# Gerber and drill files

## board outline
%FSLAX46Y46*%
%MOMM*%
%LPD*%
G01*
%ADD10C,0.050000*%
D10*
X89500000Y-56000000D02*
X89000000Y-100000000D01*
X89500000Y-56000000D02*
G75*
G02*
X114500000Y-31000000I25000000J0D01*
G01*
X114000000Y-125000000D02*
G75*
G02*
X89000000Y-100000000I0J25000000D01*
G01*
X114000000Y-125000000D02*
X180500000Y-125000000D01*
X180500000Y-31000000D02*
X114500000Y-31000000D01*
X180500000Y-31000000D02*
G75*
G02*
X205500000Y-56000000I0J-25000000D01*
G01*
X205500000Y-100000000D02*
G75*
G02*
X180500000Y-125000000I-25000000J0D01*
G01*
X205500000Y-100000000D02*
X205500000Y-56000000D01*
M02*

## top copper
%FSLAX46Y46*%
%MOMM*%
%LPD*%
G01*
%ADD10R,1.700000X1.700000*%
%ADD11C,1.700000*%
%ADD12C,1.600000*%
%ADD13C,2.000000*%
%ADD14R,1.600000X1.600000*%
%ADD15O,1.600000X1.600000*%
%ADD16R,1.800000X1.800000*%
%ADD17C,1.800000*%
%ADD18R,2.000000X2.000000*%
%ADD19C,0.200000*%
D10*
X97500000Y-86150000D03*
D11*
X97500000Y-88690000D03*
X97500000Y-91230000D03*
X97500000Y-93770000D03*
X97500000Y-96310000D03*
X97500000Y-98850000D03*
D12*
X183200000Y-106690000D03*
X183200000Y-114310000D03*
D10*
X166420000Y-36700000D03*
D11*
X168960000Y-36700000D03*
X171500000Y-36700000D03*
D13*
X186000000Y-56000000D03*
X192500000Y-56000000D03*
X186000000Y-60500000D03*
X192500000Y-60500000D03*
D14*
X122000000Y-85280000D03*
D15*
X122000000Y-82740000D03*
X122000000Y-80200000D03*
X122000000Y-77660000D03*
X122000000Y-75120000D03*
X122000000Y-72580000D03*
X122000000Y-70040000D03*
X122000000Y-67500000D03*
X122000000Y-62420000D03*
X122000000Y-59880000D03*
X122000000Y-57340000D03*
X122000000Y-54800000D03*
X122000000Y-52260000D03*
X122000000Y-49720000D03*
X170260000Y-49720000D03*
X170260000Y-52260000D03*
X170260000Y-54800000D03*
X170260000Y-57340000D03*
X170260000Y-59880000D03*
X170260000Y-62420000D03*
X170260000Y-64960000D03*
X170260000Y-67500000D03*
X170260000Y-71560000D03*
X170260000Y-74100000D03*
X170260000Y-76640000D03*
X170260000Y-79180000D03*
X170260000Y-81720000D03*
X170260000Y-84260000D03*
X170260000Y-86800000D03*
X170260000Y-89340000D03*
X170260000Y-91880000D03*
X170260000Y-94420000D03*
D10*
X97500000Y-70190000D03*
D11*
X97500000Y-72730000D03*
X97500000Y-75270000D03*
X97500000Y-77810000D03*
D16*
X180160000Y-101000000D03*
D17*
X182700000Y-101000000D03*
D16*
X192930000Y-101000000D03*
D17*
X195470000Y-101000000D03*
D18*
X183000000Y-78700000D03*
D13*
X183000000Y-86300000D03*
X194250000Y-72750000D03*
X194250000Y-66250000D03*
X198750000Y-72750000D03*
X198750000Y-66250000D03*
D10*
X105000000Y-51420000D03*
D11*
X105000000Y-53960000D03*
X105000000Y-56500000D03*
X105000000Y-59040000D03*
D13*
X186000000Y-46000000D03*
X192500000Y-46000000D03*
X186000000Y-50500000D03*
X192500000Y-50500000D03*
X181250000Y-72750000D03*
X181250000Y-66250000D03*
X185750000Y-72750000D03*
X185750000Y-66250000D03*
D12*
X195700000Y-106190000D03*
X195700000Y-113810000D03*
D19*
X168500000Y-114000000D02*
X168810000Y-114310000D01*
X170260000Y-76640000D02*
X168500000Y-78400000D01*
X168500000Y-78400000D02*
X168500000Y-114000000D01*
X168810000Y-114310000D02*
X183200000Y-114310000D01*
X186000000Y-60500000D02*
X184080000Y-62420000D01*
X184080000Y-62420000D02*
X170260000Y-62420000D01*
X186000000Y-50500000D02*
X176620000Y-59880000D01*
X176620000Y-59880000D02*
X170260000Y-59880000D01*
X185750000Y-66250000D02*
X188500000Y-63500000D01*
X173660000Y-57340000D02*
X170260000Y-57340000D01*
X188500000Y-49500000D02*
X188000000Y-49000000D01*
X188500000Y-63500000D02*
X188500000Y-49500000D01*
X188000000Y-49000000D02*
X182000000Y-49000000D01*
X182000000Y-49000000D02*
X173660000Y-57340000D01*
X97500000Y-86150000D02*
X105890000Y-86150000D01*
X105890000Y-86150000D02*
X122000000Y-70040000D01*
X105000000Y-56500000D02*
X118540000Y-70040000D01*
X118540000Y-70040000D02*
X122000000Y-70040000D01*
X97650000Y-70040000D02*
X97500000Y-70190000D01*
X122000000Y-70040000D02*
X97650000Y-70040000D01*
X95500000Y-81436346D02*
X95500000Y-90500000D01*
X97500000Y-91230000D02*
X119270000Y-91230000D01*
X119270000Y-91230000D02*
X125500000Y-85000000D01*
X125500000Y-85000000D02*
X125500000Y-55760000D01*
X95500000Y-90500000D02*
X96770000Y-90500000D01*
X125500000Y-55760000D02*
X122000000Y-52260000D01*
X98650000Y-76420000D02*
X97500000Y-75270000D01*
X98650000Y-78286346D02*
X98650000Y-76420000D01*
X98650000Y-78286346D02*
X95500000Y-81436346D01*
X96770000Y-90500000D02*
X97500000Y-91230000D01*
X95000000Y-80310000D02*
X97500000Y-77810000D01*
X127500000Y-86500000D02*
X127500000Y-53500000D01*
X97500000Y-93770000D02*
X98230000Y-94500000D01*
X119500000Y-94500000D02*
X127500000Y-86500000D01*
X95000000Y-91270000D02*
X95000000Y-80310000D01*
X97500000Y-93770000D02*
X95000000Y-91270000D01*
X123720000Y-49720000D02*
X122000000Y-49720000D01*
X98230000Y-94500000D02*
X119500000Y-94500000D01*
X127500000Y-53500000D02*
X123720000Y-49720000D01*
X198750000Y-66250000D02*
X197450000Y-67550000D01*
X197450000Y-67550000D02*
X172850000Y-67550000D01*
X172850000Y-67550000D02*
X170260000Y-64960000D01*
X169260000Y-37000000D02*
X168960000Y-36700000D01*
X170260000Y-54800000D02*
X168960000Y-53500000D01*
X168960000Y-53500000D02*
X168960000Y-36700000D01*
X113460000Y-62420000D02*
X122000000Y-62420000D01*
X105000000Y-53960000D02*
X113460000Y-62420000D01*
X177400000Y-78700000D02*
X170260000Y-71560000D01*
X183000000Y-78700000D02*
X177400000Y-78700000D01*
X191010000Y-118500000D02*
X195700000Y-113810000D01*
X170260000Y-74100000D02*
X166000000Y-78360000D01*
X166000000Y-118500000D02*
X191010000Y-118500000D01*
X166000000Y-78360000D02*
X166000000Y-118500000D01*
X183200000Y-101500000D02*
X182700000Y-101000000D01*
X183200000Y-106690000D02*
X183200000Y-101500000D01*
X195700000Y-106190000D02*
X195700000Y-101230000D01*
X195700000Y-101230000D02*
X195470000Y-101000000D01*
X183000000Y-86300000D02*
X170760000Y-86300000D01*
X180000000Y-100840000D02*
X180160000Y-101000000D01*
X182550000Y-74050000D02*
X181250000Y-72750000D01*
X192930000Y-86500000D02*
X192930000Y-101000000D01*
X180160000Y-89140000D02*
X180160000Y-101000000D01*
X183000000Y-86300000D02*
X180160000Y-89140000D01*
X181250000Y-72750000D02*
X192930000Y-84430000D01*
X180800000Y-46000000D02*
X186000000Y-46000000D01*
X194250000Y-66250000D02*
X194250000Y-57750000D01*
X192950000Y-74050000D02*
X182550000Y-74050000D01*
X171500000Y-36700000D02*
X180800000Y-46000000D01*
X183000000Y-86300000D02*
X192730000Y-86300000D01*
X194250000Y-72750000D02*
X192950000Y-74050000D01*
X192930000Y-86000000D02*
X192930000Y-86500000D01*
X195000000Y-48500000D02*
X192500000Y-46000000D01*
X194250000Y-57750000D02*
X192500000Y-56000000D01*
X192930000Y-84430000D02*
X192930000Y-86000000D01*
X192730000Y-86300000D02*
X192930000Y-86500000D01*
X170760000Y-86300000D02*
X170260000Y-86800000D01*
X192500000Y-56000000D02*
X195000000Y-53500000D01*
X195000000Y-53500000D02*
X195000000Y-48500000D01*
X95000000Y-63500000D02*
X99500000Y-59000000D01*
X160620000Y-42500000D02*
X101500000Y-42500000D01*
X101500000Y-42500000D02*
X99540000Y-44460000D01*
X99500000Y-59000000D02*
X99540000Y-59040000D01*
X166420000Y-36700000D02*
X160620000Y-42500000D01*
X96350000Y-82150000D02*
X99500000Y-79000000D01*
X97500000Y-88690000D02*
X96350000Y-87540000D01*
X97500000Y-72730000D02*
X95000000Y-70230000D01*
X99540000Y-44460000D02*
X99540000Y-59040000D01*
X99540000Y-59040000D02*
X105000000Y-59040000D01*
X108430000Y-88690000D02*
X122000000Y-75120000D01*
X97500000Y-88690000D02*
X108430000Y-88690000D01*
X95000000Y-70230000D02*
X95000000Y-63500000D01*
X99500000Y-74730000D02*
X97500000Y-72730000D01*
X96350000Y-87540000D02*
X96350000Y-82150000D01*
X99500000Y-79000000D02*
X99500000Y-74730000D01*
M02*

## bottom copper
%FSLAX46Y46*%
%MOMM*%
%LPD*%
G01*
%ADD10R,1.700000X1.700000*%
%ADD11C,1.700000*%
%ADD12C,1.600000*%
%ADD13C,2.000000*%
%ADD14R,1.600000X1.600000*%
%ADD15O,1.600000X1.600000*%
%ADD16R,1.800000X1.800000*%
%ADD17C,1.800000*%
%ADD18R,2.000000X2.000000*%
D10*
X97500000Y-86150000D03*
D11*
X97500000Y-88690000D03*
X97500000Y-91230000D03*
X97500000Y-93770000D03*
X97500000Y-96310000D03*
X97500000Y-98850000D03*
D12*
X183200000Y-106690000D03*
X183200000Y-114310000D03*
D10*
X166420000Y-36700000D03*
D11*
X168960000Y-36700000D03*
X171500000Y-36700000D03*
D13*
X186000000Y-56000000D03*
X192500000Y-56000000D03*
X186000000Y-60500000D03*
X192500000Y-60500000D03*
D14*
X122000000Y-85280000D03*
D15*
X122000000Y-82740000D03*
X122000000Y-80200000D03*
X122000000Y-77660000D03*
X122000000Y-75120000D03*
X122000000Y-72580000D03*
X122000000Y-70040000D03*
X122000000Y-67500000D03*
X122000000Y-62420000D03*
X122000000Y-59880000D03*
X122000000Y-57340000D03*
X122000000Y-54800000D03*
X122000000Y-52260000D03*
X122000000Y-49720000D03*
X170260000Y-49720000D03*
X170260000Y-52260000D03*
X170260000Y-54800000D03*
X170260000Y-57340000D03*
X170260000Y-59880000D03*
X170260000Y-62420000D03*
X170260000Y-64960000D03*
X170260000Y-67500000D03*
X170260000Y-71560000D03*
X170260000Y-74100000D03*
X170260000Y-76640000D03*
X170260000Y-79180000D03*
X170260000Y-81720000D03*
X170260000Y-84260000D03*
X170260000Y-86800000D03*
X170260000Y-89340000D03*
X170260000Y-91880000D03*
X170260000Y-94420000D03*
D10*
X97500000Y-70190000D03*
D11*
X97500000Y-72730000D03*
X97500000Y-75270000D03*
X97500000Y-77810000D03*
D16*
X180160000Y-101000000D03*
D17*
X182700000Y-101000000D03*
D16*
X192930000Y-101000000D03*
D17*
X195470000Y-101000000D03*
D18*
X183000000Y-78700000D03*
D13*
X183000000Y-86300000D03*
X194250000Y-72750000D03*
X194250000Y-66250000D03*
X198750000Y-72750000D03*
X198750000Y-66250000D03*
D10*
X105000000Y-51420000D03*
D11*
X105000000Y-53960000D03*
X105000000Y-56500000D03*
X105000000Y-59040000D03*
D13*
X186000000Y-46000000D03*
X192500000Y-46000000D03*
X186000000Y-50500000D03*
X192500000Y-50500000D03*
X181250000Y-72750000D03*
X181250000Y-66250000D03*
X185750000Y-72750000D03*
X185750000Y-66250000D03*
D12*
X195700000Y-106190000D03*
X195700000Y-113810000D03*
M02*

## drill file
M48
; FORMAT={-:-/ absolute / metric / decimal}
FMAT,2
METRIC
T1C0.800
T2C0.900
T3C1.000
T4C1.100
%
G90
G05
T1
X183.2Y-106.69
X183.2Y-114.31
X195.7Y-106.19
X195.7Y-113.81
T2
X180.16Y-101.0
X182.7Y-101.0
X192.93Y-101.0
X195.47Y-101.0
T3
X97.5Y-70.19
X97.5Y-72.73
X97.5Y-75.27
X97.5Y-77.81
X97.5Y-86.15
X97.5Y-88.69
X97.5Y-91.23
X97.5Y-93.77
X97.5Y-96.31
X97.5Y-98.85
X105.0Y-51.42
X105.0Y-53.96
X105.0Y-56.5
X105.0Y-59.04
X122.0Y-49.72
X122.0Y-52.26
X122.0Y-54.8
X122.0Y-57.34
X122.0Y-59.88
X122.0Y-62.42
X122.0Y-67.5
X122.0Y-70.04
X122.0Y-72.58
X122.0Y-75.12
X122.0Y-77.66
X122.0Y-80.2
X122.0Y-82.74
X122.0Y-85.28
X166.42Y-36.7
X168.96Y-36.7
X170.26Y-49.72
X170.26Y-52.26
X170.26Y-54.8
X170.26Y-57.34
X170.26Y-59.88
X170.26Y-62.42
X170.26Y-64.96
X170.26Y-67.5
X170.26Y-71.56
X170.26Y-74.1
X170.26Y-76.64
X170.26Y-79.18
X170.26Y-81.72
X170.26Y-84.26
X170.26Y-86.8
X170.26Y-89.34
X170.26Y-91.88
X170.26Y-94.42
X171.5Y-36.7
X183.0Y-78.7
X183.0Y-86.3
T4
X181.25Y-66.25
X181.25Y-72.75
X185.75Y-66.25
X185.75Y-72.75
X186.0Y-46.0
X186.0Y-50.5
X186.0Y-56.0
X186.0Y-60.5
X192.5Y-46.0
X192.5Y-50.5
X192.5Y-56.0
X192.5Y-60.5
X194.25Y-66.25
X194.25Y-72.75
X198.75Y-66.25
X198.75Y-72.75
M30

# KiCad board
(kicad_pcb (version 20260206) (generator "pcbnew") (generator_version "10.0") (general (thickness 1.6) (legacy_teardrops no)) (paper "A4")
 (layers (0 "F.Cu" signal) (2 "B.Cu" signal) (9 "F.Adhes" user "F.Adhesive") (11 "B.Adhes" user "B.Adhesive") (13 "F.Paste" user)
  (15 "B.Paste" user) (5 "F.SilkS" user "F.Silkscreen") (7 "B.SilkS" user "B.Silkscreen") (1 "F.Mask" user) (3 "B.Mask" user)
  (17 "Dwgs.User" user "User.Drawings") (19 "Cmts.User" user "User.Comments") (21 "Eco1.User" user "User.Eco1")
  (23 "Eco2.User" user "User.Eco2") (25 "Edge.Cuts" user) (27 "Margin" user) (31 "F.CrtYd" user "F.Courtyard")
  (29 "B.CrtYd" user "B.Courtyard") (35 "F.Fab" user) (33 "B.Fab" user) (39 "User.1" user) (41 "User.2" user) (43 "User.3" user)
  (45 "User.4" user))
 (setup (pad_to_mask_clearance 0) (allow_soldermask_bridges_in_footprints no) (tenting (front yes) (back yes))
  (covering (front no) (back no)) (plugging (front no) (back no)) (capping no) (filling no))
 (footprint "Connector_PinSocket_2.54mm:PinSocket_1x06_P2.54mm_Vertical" (layer "F.Cu") (at 97.5 86.15)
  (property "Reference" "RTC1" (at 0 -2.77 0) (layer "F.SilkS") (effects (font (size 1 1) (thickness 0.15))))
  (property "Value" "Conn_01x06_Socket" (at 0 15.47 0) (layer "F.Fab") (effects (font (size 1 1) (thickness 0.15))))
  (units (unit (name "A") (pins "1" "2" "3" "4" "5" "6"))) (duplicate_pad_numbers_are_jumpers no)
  (pad "1" thru_hole rect (at 0 0) (size 1.7 1.7) (drill 1) (layers "*.Cu" "*.Mask") (remove_unused_layers no) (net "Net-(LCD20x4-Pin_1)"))
  (pad "2" thru_hole circle (at 0 2.54) (size 1.7 1.7) (drill 1) (layers "*.Cu" "*.Mask") (remove_unused_layers no) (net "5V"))
  (pad "3" thru_hole circle (at 0 5.08) (size 1.7 1.7) (drill 1) (layers "*.Cu" "*.Mask") (remove_unused_layers no)
   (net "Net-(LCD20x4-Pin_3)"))
  (pad "4" thru_hole circle (at 0 7.62) (size 1.7 1.7) (drill 1) (layers "*.Cu" "*.Mask") (remove_unused_layers no)
   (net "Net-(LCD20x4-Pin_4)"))
  (pad "5" thru_hole circle (at 0 10.16) (size 1.7 1.7) (drill 1) (layers "*.Cu" "*.Mask") (remove_unused_layers no)
   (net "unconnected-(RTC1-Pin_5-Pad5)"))
  (pad "6" thru_hole circle (at 0 12.7) (size 1.7 1.7) (drill 1) (layers "*.Cu" "*.Mask") (remove_unused_layers no)
   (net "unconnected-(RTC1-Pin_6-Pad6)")))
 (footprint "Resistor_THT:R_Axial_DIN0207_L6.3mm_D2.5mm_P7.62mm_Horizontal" (layer "F.Cu") (at 183.2 106.69 -90)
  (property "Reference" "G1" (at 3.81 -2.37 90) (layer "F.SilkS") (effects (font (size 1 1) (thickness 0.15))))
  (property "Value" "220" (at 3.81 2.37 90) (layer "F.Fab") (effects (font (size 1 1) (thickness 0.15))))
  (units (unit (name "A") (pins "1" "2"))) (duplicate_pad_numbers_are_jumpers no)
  (pad "1" thru_hole circle (at 0 0 270) (size 1.6 1.6) (drill 0.8) (layers "*.Cu" "*.Mask") (remove_unused_layers no)
   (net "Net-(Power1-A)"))
  (pad "2" thru_hole circle (at 7.62 0 270) (size 1.6 1.6) (drill 0.8) (layers "*.Cu" "*.Mask") (remove_unused_layers no)
   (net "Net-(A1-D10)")))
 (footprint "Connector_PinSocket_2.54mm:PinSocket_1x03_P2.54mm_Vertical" (layer "F.Cu") (at 166.42 36.7 90)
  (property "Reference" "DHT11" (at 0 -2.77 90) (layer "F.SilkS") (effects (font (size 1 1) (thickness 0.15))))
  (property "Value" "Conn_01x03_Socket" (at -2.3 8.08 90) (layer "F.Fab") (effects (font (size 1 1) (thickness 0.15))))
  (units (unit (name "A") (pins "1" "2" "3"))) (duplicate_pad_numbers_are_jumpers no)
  (pad "1" thru_hole rect (at 0 0 90) (size 1.7 1.7) (drill 1) (layers "*.Cu" "*.Mask") (remove_unused_layers no) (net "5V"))
  (pad "2" thru_hole circle (at 0 2.54 90) (size 1.7 1.7) (drill 1) (layers "*.Cu" "*.Mask") (remove_unused_layers no) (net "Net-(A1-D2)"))
  (pad "3" thru_hole circle (at 0 5.08 90) (size 1.7 1.7) (drill 1) (layers "*.Cu" "*.Mask") (remove_unused_layers no)
   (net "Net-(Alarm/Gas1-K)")))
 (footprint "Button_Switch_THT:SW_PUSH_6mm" (layer "F.Cu") (at 186 56)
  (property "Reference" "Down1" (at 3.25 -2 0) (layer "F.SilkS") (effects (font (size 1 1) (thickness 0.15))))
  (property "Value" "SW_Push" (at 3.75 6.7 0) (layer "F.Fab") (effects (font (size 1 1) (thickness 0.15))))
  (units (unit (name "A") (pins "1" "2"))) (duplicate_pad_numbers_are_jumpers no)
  (pad "1" thru_hole circle (at 0 0 90) (size 2 2) (drill 1.1) (layers "*.Cu" "*.Mask") (remove_unused_layers no) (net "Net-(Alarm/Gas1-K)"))
  (pad "1" thru_hole circle (at 6.5 0 90) (size 2 2) (drill 1.1) (layers "*.Cu" "*.Mask") (remove_unused_layers no)
   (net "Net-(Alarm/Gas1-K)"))
  (pad "2" thru_hole circle (at 0 4.5 90) (size 2 2) (drill 1.1) (layers "*.Cu" "*.Mask") (remove_unused_layers no) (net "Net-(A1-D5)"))
  (pad "2" thru_hole circle (at 6.5 4.5 90) (size 2 2) (drill 1.1) (layers "*.Cu" "*.Mask") (remove_unused_layers no) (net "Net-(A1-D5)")))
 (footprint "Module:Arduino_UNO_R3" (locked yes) (layer "F.Cu") (at 122 85.28 90)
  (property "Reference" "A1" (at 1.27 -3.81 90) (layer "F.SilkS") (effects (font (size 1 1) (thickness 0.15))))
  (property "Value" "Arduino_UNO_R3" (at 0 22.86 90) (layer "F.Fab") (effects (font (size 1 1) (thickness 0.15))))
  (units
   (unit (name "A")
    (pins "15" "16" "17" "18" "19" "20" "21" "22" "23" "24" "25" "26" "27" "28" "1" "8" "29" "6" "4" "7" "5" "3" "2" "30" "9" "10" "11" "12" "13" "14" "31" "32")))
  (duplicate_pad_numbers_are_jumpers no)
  (pad "1" thru_hole rect (at 0 0 180) (size 1.6 1.6) (drill 1) (layers "*.Cu" "*.Mask") (remove_unused_layers no)
   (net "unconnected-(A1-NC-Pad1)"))
  (pad "2" thru_hole oval (at 2.54 0 180) (size 1.6 1.6) (drill 1) (layers "*.Cu" "*.Mask") (remove_unused_layers no)
   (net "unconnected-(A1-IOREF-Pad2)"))
  (pad "3" thru_hole oval (at 5.08 0 180) (size 1.6 1.6) (drill 1) (layers "*.Cu" "*.Mask") (remove_unused_layers no)
   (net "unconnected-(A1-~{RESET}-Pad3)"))
  (pad "4" thru_hole oval (at 7.62 0 180) (size 1.6 1.6) (drill 1) (layers "*.Cu" "*.Mask") (remove_unused_layers no)
   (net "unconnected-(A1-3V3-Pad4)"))
  (pad "5" thru_hole oval (at 10.16 0 180) (size 1.6 1.6) (drill 1) (layers "*.Cu" "*.Mask") (remove_unused_layers no) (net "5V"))
  (pad "6" thru_hole oval (at 12.7 0 180) (size 1.6 1.6) (drill 1) (layers "*.Cu" "*.Mask") (remove_unused_layers no) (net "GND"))
  (pad "7" thru_hole oval (at 15.24 0 180) (size 1.6 1.6) (drill 1) (layers "*.Cu" "*.Mask") (remove_unused_layers no)
   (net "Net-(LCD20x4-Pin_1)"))
  (pad "8" thru_hole oval (at 17.78 0 180) (size 1.6 1.6) (drill 1) (layers "*.Cu" "*.Mask") (remove_unused_layers no)
   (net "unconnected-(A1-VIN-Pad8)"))
  (pad "9" thru_hole oval (at 22.86 0 180) (size 1.6 1.6) (drill 1) (layers "*.Cu" "*.Mask") (remove_unused_layers no) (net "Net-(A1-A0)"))
  (pad "10" thru_hole oval (at 25.4 0 180) (size 1.6 1.6) (drill 1) (layers "*.Cu" "*.Mask") (remove_unused_layers no)
   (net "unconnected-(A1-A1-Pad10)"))
  (pad "11" thru_hole oval (at 27.94 0 180) (size 1.6 1.6) (drill 1) (layers "*.Cu" "*.Mask") (remove_unused_layers no)
   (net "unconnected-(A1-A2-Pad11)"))
  (pad "12" thru_hole oval (at 30.48 0 180) (size 1.6 1.6) (drill 1) (layers "*.Cu" "*.Mask") (remove_unused_layers no)
   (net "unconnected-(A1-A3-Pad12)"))
  (pad "13" thru_hole oval (at 33.02 0 180) (size 1.6 1.6) (drill 1) (layers "*.Cu" "*.Mask") (remove_unused_layers no)
   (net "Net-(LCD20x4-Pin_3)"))
  (pad "14" thru_hole oval (at 35.56 0 180) (size 1.6 1.6) (drill 1) (layers "*.Cu" "*.Mask") (remove_unused_layers no)
   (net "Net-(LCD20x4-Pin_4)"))
  (pad "15" thru_hole oval (at 35.56 48.26 180) (size 1.6 1.6) (drill 1) (layers "*.Cu" "*.Mask") (remove_unused_layers no)
   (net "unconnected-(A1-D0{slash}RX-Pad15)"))
  (pad "16" thru_hole oval (at 33.02 48.26 180) (size 1.6 1.6) (drill 1) (layers "*.Cu" "*.Mask") (remove_unused_layers no)
   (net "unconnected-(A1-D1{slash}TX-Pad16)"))
  (pad "17" thru_hole oval (at 30.48 48.26 180) (size 1.6 1.6) (drill 1) (layers "*.Cu" "*.Mask") (remove_unused_layers no)
   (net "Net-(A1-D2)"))
  (pad "18" thru_hole oval (at 27.94 48.26 180) (size 1.6 1.6) (drill 1) (layers "*.Cu" "*.Mask") (remove_unused_layers no)
   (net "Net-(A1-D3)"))
  (pad "19" thru_hole oval (at 25.4 48.26 180) (size 1.6 1.6) (drill 1) (layers "*.Cu" "*.Mask") (remove_unused_layers no)
   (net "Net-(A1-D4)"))
  (pad "20" thru_hole oval (at 22.86 48.26 180) (size 1.6 1.6) (drill 1) (layers "*.Cu" "*.Mask") (remove_unused_layers no)
   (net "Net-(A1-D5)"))
  (pad "21" thru_hole oval (at 20.32 48.26 180) (size 1.6 1.6) (drill 1) (layers "*.Cu" "*.Mask") (remove_unused_layers no)
   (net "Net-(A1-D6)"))
  (pad "22" thru_hole oval (at 17.78 48.26 180) (size 1.6 1.6) (drill 1) (layers "*.Cu" "*.Mask") (remove_unused_layers no)
   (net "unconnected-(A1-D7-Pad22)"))
  (pad "23" thru_hole oval (at 13.72 48.26 180) (size 1.6 1.6) (drill 1) (layers "*.Cu" "*.Mask") (remove_unused_layers no)
   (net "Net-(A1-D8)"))
  (pad "24" thru_hole oval (at 11.18 48.26 180) (size 1.6 1.6) (drill 1) (layers "*.Cu" "*.Mask") (remove_unused_layers no)
   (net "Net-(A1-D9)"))
  (pad "25" thru_hole oval (at 8.64 48.26 180) (size 1.6 1.6) (drill 1) (layers "*.Cu" "*.Mask") (remove_unused_layers no)
   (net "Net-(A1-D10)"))
  (pad "26" thru_hole oval (at 6.1 48.26 180) (size 1.6 1.6) (drill 1) (layers "*.Cu" "*.Mask") (remove_unused_layers no)
   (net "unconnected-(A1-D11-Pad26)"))
  (pad "27" thru_hole oval (at 3.56 48.26 180) (size 1.6 1.6) (drill 1) (layers "*.Cu" "*.Mask") (remove_unused_layers no)
   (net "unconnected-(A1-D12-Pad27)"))
  (pad "28" thru_hole oval (at 1.02 48.26 180) (size 1.6 1.6) (drill 1) (layers "*.Cu" "*.Mask") (remove_unused_layers no)
   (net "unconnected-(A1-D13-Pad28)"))
  (pad "29" thru_hole oval (at -1.52 48.26 180) (size 1.6 1.6) (drill 1) (layers "*.Cu" "*.Mask") (remove_unused_layers no)
   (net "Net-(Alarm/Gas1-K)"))
  (pad "30" thru_hole oval (at -4.06 48.26 180) (size 1.6 1.6) (drill 1) (layers "*.Cu" "*.Mask") (remove_unused_layers no)
   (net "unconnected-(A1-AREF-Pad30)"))
  (pad "31" thru_hole oval (at -6.6 48.26 180) (size 1.6 1.6) (drill 1) (layers "*.Cu" "*.Mask") (remove_unused_layers no)
   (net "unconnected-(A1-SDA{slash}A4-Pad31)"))
  (pad "32" thru_hole oval (at -9.14 48.26 180) (size 1.6 1.6) (drill 1) (layers "*.Cu" "*.Mask") (remove_unused_layers no)
   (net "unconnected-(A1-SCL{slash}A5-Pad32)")))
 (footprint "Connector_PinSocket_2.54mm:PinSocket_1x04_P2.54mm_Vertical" (layer "F.Cu") (at 97.5 70.19)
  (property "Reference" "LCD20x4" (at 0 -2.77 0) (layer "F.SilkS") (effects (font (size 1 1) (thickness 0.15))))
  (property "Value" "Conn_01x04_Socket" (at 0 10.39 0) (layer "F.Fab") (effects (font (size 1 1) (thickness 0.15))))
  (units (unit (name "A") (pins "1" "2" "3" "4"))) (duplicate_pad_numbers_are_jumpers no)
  (pad "1" thru_hole rect (at 0 0) (size 1.7 1.7) (drill 1) (layers "*.Cu" "*.Mask") (remove_unused_layers no) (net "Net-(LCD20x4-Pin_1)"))
  (pad "2" thru_hole circle (at 0 2.54) (size 1.7 1.7) (drill 1) (layers "*.Cu" "*.Mask") (remove_unused_layers no) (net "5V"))
  (pad "3" thru_hole circle (at 0 5.08) (size 1.7 1.7) (drill 1) (layers "*.Cu" "*.Mask") (remove_unused_layers no)
   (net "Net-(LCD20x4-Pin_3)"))
  (pad "4" thru_hole circle (at 0 7.62) (size 1.7 1.7) (drill 1) (layers "*.Cu" "*.Mask") (remove_unused_layers no)
   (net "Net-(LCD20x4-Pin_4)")))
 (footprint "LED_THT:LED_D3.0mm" (layer "F.Cu") (at 180.16 101)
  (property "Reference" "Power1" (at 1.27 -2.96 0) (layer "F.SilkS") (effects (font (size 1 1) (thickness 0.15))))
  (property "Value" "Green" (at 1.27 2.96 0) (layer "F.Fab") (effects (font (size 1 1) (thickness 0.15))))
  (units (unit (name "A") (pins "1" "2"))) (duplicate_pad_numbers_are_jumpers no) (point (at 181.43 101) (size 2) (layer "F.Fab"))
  (pad "1" thru_hole rect (at 0 0) (size 1.8 1.8) (drill 0.9) (layers "*.Cu" "*.Mask") (remove_unused_layers no) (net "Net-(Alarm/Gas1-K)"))
  (pad "2" thru_hole circle (at 2.54 0) (size 1.8 1.8) (drill 0.9) (layers "*.Cu" "*.Mask") (remove_unused_layers no) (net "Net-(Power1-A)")))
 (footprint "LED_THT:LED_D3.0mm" (layer "F.Cu") (at 192.93 101)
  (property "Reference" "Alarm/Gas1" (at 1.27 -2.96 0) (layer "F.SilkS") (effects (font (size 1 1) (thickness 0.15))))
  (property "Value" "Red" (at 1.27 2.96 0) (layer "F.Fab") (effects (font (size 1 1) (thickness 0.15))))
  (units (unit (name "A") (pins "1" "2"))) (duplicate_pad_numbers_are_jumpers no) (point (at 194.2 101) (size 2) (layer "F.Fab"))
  (pad "1" thru_hole rect (at 0 0) (size 1.8 1.8) (drill 0.9) (layers "*.Cu" "*.Mask") (remove_unused_layers no) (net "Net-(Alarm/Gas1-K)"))
  (pad "2" thru_hole circle (at 2.54 0) (size 1.8 1.8) (drill 0.9) (layers "*.Cu" "*.Mask") (remove_unused_layers no)
   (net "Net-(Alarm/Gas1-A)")))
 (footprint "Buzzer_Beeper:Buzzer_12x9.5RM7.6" (layer "F.Cu") (at 183 78.7 -90)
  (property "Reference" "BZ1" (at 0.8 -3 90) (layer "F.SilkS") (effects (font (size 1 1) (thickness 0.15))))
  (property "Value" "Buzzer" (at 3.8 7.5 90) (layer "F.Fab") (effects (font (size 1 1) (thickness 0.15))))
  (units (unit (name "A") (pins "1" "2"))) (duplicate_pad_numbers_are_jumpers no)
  (pad "1" thru_hole rect (at 0 0 270) (size 2 2) (drill 1) (layers "*.Cu" "*.Mask") (remove_unused_layers no) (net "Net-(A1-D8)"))
  (pad "2" thru_hole circle (at 7.6 0 270) (size 2 2) (drill 1) (layers "*.Cu" "*.Mask") (remove_unused_layers no)
   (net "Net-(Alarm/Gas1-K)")))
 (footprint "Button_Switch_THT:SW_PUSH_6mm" (layer "F.Cu") (at 194.25 72.75 90)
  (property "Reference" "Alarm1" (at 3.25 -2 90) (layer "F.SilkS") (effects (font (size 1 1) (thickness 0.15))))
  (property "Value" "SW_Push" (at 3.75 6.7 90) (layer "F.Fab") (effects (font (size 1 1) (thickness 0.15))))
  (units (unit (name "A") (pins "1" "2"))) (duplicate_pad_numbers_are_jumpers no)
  (pad "1" thru_hole circle (at 0 0 180) (size 2 2) (drill 1.1) (layers "*.Cu" "*.Mask") (remove_unused_layers no)
   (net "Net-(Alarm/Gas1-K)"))
  (pad "1" thru_hole circle (at 6.5 0 180) (size 2 2) (drill 1.1) (layers "*.Cu" "*.Mask") (remove_unused_layers no)
   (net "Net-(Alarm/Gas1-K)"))
  (pad "2" thru_hole circle (at 0 4.5 180) (size 2 2) (drill 1.1) (layers "*.Cu" "*.Mask") (remove_unused_layers no) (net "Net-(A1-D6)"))
  (pad "2" thru_hole circle (at 6.5 4.5 180) (size 2 2) (drill 1.1) (layers "*.Cu" "*.Mask") (remove_unused_layers no) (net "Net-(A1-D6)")))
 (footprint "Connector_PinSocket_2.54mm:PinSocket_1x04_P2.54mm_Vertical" (layer "F.Cu") (at 105 51.42)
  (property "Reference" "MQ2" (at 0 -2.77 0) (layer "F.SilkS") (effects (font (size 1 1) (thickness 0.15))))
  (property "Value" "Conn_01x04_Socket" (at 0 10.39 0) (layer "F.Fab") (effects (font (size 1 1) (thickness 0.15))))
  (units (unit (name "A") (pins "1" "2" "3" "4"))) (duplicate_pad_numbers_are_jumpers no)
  (pad "1" thru_hole rect (at 0 0) (size 1.7 1.7) (drill 1) (layers "*.Cu" "*.Mask") (remove_unused_layers no)
   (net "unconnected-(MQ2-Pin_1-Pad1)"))
  (pad "2" thru_hole circle (at 0 2.54) (size 1.7 1.7) (drill 1) (layers "*.Cu" "*.Mask") (remove_unused_layers no) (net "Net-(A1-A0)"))
  (pad "3" thru_hole circle (at 0 5.08) (size 1.7 1.7) (drill 1) (layers "*.Cu" "*.Mask") (remove_unused_layers no)
   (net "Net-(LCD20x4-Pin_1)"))
  (pad "4" thru_hole circle (at 0 7.62) (size 1.7 1.7) (drill 1) (layers "*.Cu" "*.Mask") (remove_unused_layers no) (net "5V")))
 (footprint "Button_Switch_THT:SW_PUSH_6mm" (layer "F.Cu") (at 186 46)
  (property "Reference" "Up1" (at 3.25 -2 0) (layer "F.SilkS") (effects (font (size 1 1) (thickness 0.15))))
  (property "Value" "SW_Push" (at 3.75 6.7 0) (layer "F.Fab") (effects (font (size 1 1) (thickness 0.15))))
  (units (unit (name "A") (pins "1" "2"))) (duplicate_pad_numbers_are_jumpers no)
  (pad "1" thru_hole circle (at 0 0 90) (size 2 2) (drill 1.1) (layers "*.Cu" "*.Mask") (remove_unused_layers no) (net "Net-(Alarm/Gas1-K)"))
  (pad "1" thru_hole circle (at 6.5 0 90) (size 2 2) (drill 1.1) (layers "*.Cu" "*.Mask") (remove_unused_layers no)
   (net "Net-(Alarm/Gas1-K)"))
  (pad "2" thru_hole circle (at 0 4.5 90) (size 2 2) (drill 1.1) (layers "*.Cu" "*.Mask") (remove_unused_layers no) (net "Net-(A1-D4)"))
  (pad "2" thru_hole circle (at 6.5 4.5 90) (size 2 2) (drill 1.1) (layers "*.Cu" "*.Mask") (remove_unused_layers no) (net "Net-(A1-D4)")))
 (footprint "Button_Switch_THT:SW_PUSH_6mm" (layer "F.Cu") (at 181.25 72.75 90)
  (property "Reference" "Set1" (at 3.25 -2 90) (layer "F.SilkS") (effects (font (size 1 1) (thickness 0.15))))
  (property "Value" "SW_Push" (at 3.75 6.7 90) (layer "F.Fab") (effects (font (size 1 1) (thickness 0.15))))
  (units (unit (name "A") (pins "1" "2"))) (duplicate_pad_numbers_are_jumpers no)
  (pad "1" thru_hole circle (at 0 0 180) (size 2 2) (drill 1.1) (layers "*.Cu" "*.Mask") (remove_unused_layers no)
   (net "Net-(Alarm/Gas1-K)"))
  (pad "1" thru_hole circle (at 6.5 0 180) (size 2 2) (drill 1.1) (layers "*.Cu" "*.Mask") (remove_unused_layers no)
   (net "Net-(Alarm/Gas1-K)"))
  (pad "2" thru_hole circle (at 0 4.5 180) (size 2 2) (drill 1.1) (layers "*.Cu" "*.Mask") (remove_unused_layers no) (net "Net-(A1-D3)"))
  (pad "2" thru_hole circle (at 6.5 4.5 180) (size 2 2) (drill 1.1) (layers "*.Cu" "*.Mask") (remove_unused_layers no) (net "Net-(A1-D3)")))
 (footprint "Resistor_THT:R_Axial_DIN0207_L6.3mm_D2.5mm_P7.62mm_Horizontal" (layer "F.Cu") (at 195.7 106.19 -90)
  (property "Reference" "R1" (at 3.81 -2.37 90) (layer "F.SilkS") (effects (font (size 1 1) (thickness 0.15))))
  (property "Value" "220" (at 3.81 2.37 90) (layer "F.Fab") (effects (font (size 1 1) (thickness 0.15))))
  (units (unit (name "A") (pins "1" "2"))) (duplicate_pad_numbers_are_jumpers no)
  (pad "1" thru_hole circle (at 0 0 270) (size 1.6 1.6) (drill 0.8) (layers "*.Cu" "*.Mask") (remove_unused_layers no)
   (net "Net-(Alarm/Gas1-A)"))
  (pad "2" thru_hole circle (at 7.62 0 270) (size 1.6 1.6) (drill 0.8) (layers "*.Cu" "*.Mask") (remove_unused_layers no)
   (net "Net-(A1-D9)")))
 (gr_line (start 89.5 56) (end 89 100) (stroke (width 0.05) (type default)) (layer "Edge.Cuts"))
 (gr_arc (start 89.5 56) (mid 96.82233 38.32233) (end 114.5 31) (stroke (width 0.05) (type default)) (layer "Edge.Cuts"))
 (gr_arc (start 114 125) (mid 96.32233 117.67767) (end 89 100) (stroke (width 0.05) (type default)) (layer "Edge.Cuts"))
 (gr_line (start 114 125) (end 180.5 125) (stroke (width 0.05) (type default)) (layer "Edge.Cuts"))
 (gr_line (start 180.5 31) (end 114.5 31) (stroke (width 0.05) (type default)) (layer "Edge.Cuts"))
 (gr_arc (start 180.5 31) (mid 198.17767 38.32233) (end 205.5 56) (stroke (width 0.05) (type default)) (layer "Edge.Cuts"))
 (gr_arc (start 205.5 100) (mid 198.17767 117.67767) (end 180.5 125) (stroke (width 0.05) (type default)) (layer "Edge.Cuts"))
 (gr_line (start 205.5 100) (end 205.5 56) (stroke (width 0.05) (type default)) (layer "Edge.Cuts"))
 (segment (start 168.5 114) (end 168.81 114.31) (width 0.2) (layer "F.Cu") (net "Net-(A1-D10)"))
 (segment (start 170.26 76.64) (end 168.5 78.4) (width 0.2) (layer "F.Cu") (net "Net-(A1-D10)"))
 (segment (start 168.5 78.4) (end 168.5 114) (width 0.2) (layer "F.Cu") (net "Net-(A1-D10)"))
 (segment (start 168.81 114.31) (end 183.2 114.31) (width 0.2) (layer "F.Cu") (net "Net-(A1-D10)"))
 (segment (start 186 60.5) (end 184.08 62.42) (width 0.2) (layer "F.Cu") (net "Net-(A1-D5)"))
 (segment (start 184.08 62.42) (end 170.26 62.42) (width 0.2) (layer "F.Cu") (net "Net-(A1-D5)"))
 (segment (start 186 50.5) (end 176.62 59.88) (width 0.2) (layer "F.Cu") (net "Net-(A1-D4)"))
 (segment (start 176.62 59.88) (end 170.26 59.88) (width 0.2) (layer "F.Cu") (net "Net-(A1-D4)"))
 (segment (start 185.75 66.25) (end 188.5 63.5) (width 0.2) (layer "F.Cu") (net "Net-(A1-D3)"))
 (segment (start 173.66 57.34) (end 170.26 57.34) (width 0.2) (layer "F.Cu") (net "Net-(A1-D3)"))
 (segment (start 188.5 49.5) (end 188 49) (width 0.2) (layer "F.Cu") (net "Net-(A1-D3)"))
 (segment (start 188.5 63.5) (end 188.5 49.5) (width 0.2) (layer "F.Cu") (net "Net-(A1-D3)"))
 (segment (start 188 49) (end 182 49) (width 0.2) (layer "F.Cu") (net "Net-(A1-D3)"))
 (segment (start 182 49) (end 173.66 57.34) (width 0.2) (layer "F.Cu") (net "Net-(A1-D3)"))
 (segment (start 97.5 86.15) (end 105.89 86.15) (width 0.2) (layer "F.Cu") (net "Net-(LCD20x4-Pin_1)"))
 (segment (start 105.89 86.15) (end 122 70.04) (width 0.2) (layer "F.Cu") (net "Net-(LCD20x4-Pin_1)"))
 (segment (start 105 56.5) (end 118.54 70.04) (width 0.2) (layer "F.Cu") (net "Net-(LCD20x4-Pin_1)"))
 (segment (start 118.54 70.04) (end 122 70.04) (width 0.2) (layer "F.Cu") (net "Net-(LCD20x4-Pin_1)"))
 (segment (start 97.65 70.04) (end 97.5 70.19) (width 0.2) (layer "F.Cu") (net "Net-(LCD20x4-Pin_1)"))
 (segment (start 122 70.04) (end 97.65 70.04) (width 0.2) (layer "F.Cu") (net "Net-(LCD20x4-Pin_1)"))
 (segment (start 95.5 81.436346) (end 95.5 90.5) (width 0.2) (layer "F.Cu") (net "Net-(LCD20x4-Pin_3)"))
 (segment (start 97.5 91.23) (end 119.27 91.23) (width 0.2) (layer "F.Cu") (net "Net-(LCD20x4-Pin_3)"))
 (segment (start 119.27 91.23) (end 125.5 85) (width 0.2) (layer "F.Cu") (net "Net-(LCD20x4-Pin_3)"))
 (segment (start 125.5 85) (end 125.5 55.76) (width 0.2) (layer "F.Cu") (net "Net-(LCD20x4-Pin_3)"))
 (segment (start 95.5 90.5) (end 96.77 90.5) (width 0.2) (layer "F.Cu") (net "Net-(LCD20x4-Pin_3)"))
 (segment (start 125.5 55.76) (end 122 52.26) (width 0.2) (layer "F.Cu") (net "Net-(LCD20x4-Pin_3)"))
 (segment (start 98.65 76.42) (end 97.5 75.27) (width 0.2) (layer "F.Cu") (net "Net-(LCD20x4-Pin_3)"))
 (segment (start 98.65 78.286346) (end 98.65 76.42) (width 0.2) (layer "F.Cu") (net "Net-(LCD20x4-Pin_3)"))
 (segment (start 98.65 78.286346) (end 95.5 81.436346) (width 0.2) (layer "F.Cu") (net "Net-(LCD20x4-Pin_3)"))
 (segment (start 96.77 90.5) (end 97.5 91.23) (width 0.2) (layer "F.Cu") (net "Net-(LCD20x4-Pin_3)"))
 (segment (start 95 80.31) (end 97.5 77.81) (width 0.2) (layer "F.Cu") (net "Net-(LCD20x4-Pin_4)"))
 (segment (start 127.5 86.5) (end 127.5 53.5) (width 0.2) (layer "F.Cu") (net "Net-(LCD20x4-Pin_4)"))
 (segment (start 97.5 93.77) (end 98.23 94.5) (width 0.2) (layer "F.Cu") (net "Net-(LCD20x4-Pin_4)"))
 (segment (start 119.5 94.5) (end 127.5 86.5) (width 0.2) (layer "F.Cu") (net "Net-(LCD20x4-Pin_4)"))
 (segment (start 95 91.27) (end 95 80.31) (width 0.2) (layer "F.Cu") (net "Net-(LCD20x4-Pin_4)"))
 (segment (start 97.5 93.77) (end 95 91.27) (width 0.2) (layer "F.Cu") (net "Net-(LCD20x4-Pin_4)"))
 (segment (start 123.72 49.72) (end 122 49.72) (width 0.2) (layer "F.Cu") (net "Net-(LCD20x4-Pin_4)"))
 (segment (start 98.23 94.5) (end 119.5 94.5) (width 0.2) (layer "F.Cu") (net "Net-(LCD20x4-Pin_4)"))
 (segment (start 127.5 53.5) (end 123.72 49.72) (width 0.2) (layer "F.Cu") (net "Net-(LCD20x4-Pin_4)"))
 (segment (start 198.75 66.25) (end 197.45 67.55) (width 0.2) (layer "F.Cu") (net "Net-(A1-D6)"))
 (segment (start 197.45 67.55) (end 172.85 67.55) (width 0.2) (layer "F.Cu") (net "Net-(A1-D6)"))
 (segment (start 172.85 67.55) (end 170.26 64.96) (width 0.2) (layer "F.Cu") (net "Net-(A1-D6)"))
 (segment (start 169.26 37) (end 168.96 36.7) (width 0.2) (layer "F.Cu") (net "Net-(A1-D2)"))
 (segment (start 170.26 54.8) (end 168.96 53.5) (width 0.2) (layer "F.Cu") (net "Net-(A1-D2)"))
 (segment (start 168.96 53.5) (end 168.96 36.7) (width 0.2) (layer "F.Cu") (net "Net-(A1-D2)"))
 (segment (start 113.46 62.42) (end 122 62.42) (width 0.2) (layer "F.Cu") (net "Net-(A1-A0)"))
 (segment (start 105 53.96) (end 113.46 62.42) (width 0.2) (layer "F.Cu") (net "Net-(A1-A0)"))
 (segment (start 177.4 78.7) (end 170.26 71.56) (width 0.2) (layer "F.Cu") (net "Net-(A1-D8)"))
 (segment (start 183 78.7) (end 177.4 78.7) (width 0.2) (layer "F.Cu") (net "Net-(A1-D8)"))
 (segment (start 191.01 118.5) (end 195.7 113.81) (width 0.2) (layer "F.Cu") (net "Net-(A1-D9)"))
 (segment (start 170.26 74.1) (end 166 78.36) (width 0.2) (layer "F.Cu") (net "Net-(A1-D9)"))
 (segment (start 166 118.5) (end 191.01 118.5) (width 0.2) (layer "F.Cu") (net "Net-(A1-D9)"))
 (segment (start 166 78.36) (end 166 118.5) (width 0.2) (layer "F.Cu") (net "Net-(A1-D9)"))
 (segment (start 183.2 101.5) (end 182.7 101) (width 0.2) (layer "F.Cu") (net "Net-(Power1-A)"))
 (segment (start 183.2 106.69) (end 183.2 101.5) (width 0.2) (layer "F.Cu") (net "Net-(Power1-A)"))
 (segment (start 195.7 106.19) (end 195.7 101.23) (width 0.2) (layer "F.Cu") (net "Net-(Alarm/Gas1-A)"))
 (segment (start 195.7 101.23) (end 195.47 101) (width 0.2) (layer "F.Cu") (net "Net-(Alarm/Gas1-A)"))
 (segment (start 183 86.3) (end 170.76 86.3) (width 0.2) (layer "F.Cu") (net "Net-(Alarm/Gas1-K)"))
 (segment (start 180 100.84) (end 180.16 101) (width 0.2) (layer "F.Cu") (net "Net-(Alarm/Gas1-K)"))
 (segment (start 182.55 74.05) (end 181.25 72.75) (width 0.2) (layer "F.Cu") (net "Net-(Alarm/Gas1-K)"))
 (segment (start 192.93 86.5) (end 192.93 101) (width 0.2) (layer "F.Cu") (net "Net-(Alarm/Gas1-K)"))
 (segment (start 180.16 89.14) (end 180.16 101) (width 0.2) (layer "F.Cu") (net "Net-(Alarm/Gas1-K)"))
 (segment (start 183 86.3) (end 180.16 89.14) (width 0.2) (layer "F.Cu") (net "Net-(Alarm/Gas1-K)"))
 (segment (start 181.25 72.75) (end 192.93 84.43) (width 0.2) (layer "F.Cu") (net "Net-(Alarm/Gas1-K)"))
 (segment (start 180.8 46) (end 186 46) (width 0.2) (layer "F.Cu") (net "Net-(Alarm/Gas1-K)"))
 (segment (start 194.25 66.25) (end 194.25 57.75) (width 0.2) (layer "F.Cu") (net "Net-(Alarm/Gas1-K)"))
 (segment (start 192.95 74.05) (end 182.55 74.05) (width 0.2) (layer "F.Cu") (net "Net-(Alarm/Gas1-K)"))
 (segment (start 171.5 36.7) (end 180.8 46) (width 0.2) (layer "F.Cu") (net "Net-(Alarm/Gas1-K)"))
 (segment (start 183 86.3) (end 192.73 86.3) (width 0.2) (layer "F.Cu") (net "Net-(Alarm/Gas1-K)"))
 (segment (start 194.25 72.75) (end 192.95 74.05) (width 0.2) (layer "F.Cu") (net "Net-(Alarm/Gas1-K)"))
 (segment (start 192.93 86) (end 192.93 86.5) (width 0.2) (layer "F.Cu") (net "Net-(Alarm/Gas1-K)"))
 (segment (start 195 48.5) (end 192.5 46) (width 0.2) (layer "F.Cu") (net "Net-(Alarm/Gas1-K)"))
 (segment (start 194.25 57.75) (end 192.5 56) (width 0.2) (layer "F.Cu") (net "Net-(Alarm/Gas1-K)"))
 (segment (start 192.93 84.43) (end 192.93 86) (width 0.2) (layer "F.Cu") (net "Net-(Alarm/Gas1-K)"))
 (segment (start 192.73 86.3) (end 192.93 86.5) (width 0.2) (layer "F.Cu") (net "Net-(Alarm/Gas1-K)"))
 (segment (start 170.76 86.3) (end 170.26 86.8) (width 0.2) (layer "F.Cu") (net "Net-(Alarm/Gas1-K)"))
 (segment (start 192.5 56) (end 195 53.5) (width 0.2) (layer "F.Cu") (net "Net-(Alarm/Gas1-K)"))
 (segment (start 195 53.5) (end 195 48.5) (width 0.2) (layer "F.Cu") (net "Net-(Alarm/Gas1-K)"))
 (segment (start 95 63.5) (end 99.5 59) (width 0.2) (layer "F.Cu") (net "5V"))
 (segment (start 160.62 42.5) (end 101.5 42.5) (width 0.2) (layer "F.Cu") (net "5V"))
 (segment (start 101.5 42.5) (end 99.54 44.46) (width 0.2) (layer "F.Cu") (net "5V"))
 (segment (start 99.5 59) (end 99.54 59.04) (width 0.2) (layer "F.Cu") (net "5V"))
 (segment (start 166.42 36.7) (end 160.62 42.5) (width 0.2) (layer "F.Cu") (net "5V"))
 (segment (start 96.35 82.15) (end 99.5 79) (width 0.2) (layer "F.Cu") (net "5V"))
 (segment (start 97.5 88.69) (end 96.35 87.54) (width 0.2) (layer "F.Cu") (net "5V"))
 (segment (start 97.5 72.73) (end 95 70.23) (width 0.2) (layer "F.Cu") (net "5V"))
 (segment (start 99.54 44.46) (end 99.54 59.04) (width 0.2) (layer "F.Cu") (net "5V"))
 (segment (start 99.54 59.04) (end 105 59.04) (width 0.2) (layer "F.Cu") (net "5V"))
 (segment (start 108.43 88.69) (end 122 75.12) (width 0.2) (layer "F.Cu") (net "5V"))
 (segment (start 97.5 88.69) (end 108.43 88.69) (width 0.2) (layer "F.Cu") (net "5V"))
 (segment (start 95 70.23) (end 95 63.5) (width 0.2) (layer "F.Cu") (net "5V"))
 (segment (start 99.5 74.73) (end 97.5 72.73) (width 0.2) (layer "F.Cu") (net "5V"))
 (segment (start 96.35 87.54) (end 96.35 82.15) (width 0.2) (layer "F.Cu") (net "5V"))
 (segment (start 99.5 79) (end 99.5 74.73) (width 0.2) (layer "F.Cu") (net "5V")))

